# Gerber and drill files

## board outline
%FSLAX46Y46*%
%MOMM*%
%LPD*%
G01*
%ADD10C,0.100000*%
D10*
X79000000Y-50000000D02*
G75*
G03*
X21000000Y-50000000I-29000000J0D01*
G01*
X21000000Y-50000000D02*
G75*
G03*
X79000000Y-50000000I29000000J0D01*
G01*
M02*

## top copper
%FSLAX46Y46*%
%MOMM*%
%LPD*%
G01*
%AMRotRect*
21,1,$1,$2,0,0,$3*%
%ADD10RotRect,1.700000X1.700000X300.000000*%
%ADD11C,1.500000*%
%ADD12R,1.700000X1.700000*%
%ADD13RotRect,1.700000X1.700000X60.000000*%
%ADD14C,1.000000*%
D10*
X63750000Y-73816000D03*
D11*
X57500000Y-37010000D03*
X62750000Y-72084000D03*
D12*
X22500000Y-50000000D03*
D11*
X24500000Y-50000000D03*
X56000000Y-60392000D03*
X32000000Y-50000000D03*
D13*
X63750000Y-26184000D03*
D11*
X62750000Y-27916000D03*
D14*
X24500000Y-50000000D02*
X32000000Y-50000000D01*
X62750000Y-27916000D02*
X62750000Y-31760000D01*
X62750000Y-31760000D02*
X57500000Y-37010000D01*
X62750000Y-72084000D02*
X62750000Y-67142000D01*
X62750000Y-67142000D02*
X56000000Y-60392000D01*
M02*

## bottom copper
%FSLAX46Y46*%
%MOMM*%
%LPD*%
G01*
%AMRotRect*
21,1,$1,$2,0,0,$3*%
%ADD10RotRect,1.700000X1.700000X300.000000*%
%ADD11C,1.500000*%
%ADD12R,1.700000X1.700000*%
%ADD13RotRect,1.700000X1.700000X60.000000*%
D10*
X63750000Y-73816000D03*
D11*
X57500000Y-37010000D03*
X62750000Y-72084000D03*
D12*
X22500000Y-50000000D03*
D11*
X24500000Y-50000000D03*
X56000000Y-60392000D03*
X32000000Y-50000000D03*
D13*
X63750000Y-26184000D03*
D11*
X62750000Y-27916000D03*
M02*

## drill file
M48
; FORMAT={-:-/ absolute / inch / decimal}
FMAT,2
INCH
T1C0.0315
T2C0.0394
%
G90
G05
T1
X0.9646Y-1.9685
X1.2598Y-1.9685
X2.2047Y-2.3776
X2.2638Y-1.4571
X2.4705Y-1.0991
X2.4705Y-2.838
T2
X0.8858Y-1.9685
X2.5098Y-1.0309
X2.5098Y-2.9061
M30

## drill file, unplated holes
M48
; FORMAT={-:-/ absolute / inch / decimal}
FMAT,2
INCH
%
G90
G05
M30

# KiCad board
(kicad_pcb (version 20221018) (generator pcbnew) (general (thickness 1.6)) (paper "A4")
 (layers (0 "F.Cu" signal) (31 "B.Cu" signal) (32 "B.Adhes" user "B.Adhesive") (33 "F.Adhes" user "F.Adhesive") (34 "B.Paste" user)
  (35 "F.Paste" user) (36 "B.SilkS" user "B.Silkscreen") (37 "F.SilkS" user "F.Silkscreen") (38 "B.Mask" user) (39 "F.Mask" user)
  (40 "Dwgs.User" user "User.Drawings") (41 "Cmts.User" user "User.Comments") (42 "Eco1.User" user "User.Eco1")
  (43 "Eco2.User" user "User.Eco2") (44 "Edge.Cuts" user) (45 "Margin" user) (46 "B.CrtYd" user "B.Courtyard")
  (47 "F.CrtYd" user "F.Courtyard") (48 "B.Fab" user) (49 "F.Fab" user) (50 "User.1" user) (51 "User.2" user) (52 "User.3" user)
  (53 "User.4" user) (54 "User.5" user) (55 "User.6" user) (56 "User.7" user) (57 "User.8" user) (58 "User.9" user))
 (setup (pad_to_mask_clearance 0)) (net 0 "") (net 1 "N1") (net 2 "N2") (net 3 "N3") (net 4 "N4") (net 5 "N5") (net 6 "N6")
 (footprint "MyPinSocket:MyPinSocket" (layer "F.Cu") (at 63.75 73.816 -60)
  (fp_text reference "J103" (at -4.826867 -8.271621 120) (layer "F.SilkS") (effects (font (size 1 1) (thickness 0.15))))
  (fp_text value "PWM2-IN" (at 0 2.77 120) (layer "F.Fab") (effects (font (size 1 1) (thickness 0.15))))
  (pad "1" thru_hole rect (at 0 0 300) (size 1.7 1.7) (drill 1) (layers "*.Cu" "*.Mask") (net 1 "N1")))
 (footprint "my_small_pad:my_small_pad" (layer "F.Cu") (at 57.5 37.01)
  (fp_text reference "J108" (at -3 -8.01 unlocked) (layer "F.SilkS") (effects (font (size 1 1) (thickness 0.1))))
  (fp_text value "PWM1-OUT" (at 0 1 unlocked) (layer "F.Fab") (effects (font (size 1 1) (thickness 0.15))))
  (pad "1" thru_hole circle (at 0 0) (size 1.5 1.5) (drill 0.8) (layers "*.Cu" "*.Mask") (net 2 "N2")))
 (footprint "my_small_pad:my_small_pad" (layer "F.Cu") (at 62.75 72.084)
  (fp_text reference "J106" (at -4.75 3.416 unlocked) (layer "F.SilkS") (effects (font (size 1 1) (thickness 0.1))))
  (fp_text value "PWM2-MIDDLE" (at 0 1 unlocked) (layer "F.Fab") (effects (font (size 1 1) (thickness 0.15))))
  (pad "1" thru_hole circle (at 0 0) (size 1.5 1.5) (drill 0.8) (layers "*.Cu" "*.Mask") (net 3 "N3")))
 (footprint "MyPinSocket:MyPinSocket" (layer "F.Cu") (at 22.5 50)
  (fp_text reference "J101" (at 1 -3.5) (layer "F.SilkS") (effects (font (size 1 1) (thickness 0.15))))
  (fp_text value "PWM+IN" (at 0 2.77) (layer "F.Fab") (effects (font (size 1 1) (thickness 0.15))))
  (pad "1" thru_hole rect (at 0 0) (size 1.7 1.7) (drill 1) (layers "*.Cu" "*.Mask") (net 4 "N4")))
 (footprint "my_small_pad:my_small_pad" (layer "F.Cu") (at 24.5 50)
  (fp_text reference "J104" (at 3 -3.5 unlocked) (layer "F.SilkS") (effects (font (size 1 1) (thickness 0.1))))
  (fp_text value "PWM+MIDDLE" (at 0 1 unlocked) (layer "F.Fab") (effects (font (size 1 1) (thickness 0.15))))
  (pad "1" thru_hole circle (at 0 0) (size 1.5 1.5) (drill 0.8) (layers "*.Cu" "*.Mask") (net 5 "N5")))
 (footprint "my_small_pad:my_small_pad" (layer "F.Cu") (at 56 60.392)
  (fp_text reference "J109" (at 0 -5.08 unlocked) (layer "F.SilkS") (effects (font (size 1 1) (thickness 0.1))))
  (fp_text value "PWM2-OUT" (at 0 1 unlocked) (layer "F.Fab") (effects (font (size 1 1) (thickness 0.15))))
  (pad "1" thru_hole circle (at 0 0) (size 1.5 1.5) (drill 0.8) (layers "*.Cu" "*.Mask") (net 3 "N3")))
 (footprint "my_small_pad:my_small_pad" (layer "F.Cu") (at 32 50)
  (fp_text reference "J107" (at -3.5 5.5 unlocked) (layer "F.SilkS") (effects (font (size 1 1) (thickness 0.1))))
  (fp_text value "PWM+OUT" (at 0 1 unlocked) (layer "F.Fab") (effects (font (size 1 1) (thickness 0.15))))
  (pad "1" thru_hole circle (at 0 0) (size 1.5 1.5) (drill 0.8) (layers "*.Cu" "*.Mask") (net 5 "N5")))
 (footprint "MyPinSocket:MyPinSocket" (layer "F.Cu") (at 63.75 26.184 60)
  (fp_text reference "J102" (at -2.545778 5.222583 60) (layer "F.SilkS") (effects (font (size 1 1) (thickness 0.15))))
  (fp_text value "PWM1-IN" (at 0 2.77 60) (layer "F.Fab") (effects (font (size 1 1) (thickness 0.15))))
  (pad "1" thru_hole rect (at 0 0 60) (size 1.7 1.7) (drill 1) (layers "*.Cu" "*.Mask") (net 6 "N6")))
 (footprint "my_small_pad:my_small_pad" (layer "F.Cu") (at 62.75 27.916)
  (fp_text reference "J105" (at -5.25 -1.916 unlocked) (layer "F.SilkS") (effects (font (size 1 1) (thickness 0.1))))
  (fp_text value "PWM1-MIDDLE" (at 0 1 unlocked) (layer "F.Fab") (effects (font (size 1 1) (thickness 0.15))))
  (pad "1" thru_hole circle (at 0 0) (size 1.5 1.5) (drill 0.8) (layers "*.Cu" "*.Mask") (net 2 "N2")))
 (gr_circle (center 50 50) (end 79 50) (stroke (width 0.1) (type default)) (fill none) (layer "Edge.Cuts"))
 (segment (start 24.5 50) (end 32 50) (width 1) (layer "F.Cu") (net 5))
 (segment (start 62.75 27.916) (end 62.75 31.76) (width 1) (layer "F.Cu") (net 2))
 (segment (start 62.75 31.76) (end 57.5 37.01) (width 1) (layer "F.Cu") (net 2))
 (segment (start 62.75 72.084) (end 62.75 67.142) (width 1) (layer "F.Cu") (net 3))
 (segment (start 62.75 67.142) (end 56 60.392) (width 1) (layer "F.Cu") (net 3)))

